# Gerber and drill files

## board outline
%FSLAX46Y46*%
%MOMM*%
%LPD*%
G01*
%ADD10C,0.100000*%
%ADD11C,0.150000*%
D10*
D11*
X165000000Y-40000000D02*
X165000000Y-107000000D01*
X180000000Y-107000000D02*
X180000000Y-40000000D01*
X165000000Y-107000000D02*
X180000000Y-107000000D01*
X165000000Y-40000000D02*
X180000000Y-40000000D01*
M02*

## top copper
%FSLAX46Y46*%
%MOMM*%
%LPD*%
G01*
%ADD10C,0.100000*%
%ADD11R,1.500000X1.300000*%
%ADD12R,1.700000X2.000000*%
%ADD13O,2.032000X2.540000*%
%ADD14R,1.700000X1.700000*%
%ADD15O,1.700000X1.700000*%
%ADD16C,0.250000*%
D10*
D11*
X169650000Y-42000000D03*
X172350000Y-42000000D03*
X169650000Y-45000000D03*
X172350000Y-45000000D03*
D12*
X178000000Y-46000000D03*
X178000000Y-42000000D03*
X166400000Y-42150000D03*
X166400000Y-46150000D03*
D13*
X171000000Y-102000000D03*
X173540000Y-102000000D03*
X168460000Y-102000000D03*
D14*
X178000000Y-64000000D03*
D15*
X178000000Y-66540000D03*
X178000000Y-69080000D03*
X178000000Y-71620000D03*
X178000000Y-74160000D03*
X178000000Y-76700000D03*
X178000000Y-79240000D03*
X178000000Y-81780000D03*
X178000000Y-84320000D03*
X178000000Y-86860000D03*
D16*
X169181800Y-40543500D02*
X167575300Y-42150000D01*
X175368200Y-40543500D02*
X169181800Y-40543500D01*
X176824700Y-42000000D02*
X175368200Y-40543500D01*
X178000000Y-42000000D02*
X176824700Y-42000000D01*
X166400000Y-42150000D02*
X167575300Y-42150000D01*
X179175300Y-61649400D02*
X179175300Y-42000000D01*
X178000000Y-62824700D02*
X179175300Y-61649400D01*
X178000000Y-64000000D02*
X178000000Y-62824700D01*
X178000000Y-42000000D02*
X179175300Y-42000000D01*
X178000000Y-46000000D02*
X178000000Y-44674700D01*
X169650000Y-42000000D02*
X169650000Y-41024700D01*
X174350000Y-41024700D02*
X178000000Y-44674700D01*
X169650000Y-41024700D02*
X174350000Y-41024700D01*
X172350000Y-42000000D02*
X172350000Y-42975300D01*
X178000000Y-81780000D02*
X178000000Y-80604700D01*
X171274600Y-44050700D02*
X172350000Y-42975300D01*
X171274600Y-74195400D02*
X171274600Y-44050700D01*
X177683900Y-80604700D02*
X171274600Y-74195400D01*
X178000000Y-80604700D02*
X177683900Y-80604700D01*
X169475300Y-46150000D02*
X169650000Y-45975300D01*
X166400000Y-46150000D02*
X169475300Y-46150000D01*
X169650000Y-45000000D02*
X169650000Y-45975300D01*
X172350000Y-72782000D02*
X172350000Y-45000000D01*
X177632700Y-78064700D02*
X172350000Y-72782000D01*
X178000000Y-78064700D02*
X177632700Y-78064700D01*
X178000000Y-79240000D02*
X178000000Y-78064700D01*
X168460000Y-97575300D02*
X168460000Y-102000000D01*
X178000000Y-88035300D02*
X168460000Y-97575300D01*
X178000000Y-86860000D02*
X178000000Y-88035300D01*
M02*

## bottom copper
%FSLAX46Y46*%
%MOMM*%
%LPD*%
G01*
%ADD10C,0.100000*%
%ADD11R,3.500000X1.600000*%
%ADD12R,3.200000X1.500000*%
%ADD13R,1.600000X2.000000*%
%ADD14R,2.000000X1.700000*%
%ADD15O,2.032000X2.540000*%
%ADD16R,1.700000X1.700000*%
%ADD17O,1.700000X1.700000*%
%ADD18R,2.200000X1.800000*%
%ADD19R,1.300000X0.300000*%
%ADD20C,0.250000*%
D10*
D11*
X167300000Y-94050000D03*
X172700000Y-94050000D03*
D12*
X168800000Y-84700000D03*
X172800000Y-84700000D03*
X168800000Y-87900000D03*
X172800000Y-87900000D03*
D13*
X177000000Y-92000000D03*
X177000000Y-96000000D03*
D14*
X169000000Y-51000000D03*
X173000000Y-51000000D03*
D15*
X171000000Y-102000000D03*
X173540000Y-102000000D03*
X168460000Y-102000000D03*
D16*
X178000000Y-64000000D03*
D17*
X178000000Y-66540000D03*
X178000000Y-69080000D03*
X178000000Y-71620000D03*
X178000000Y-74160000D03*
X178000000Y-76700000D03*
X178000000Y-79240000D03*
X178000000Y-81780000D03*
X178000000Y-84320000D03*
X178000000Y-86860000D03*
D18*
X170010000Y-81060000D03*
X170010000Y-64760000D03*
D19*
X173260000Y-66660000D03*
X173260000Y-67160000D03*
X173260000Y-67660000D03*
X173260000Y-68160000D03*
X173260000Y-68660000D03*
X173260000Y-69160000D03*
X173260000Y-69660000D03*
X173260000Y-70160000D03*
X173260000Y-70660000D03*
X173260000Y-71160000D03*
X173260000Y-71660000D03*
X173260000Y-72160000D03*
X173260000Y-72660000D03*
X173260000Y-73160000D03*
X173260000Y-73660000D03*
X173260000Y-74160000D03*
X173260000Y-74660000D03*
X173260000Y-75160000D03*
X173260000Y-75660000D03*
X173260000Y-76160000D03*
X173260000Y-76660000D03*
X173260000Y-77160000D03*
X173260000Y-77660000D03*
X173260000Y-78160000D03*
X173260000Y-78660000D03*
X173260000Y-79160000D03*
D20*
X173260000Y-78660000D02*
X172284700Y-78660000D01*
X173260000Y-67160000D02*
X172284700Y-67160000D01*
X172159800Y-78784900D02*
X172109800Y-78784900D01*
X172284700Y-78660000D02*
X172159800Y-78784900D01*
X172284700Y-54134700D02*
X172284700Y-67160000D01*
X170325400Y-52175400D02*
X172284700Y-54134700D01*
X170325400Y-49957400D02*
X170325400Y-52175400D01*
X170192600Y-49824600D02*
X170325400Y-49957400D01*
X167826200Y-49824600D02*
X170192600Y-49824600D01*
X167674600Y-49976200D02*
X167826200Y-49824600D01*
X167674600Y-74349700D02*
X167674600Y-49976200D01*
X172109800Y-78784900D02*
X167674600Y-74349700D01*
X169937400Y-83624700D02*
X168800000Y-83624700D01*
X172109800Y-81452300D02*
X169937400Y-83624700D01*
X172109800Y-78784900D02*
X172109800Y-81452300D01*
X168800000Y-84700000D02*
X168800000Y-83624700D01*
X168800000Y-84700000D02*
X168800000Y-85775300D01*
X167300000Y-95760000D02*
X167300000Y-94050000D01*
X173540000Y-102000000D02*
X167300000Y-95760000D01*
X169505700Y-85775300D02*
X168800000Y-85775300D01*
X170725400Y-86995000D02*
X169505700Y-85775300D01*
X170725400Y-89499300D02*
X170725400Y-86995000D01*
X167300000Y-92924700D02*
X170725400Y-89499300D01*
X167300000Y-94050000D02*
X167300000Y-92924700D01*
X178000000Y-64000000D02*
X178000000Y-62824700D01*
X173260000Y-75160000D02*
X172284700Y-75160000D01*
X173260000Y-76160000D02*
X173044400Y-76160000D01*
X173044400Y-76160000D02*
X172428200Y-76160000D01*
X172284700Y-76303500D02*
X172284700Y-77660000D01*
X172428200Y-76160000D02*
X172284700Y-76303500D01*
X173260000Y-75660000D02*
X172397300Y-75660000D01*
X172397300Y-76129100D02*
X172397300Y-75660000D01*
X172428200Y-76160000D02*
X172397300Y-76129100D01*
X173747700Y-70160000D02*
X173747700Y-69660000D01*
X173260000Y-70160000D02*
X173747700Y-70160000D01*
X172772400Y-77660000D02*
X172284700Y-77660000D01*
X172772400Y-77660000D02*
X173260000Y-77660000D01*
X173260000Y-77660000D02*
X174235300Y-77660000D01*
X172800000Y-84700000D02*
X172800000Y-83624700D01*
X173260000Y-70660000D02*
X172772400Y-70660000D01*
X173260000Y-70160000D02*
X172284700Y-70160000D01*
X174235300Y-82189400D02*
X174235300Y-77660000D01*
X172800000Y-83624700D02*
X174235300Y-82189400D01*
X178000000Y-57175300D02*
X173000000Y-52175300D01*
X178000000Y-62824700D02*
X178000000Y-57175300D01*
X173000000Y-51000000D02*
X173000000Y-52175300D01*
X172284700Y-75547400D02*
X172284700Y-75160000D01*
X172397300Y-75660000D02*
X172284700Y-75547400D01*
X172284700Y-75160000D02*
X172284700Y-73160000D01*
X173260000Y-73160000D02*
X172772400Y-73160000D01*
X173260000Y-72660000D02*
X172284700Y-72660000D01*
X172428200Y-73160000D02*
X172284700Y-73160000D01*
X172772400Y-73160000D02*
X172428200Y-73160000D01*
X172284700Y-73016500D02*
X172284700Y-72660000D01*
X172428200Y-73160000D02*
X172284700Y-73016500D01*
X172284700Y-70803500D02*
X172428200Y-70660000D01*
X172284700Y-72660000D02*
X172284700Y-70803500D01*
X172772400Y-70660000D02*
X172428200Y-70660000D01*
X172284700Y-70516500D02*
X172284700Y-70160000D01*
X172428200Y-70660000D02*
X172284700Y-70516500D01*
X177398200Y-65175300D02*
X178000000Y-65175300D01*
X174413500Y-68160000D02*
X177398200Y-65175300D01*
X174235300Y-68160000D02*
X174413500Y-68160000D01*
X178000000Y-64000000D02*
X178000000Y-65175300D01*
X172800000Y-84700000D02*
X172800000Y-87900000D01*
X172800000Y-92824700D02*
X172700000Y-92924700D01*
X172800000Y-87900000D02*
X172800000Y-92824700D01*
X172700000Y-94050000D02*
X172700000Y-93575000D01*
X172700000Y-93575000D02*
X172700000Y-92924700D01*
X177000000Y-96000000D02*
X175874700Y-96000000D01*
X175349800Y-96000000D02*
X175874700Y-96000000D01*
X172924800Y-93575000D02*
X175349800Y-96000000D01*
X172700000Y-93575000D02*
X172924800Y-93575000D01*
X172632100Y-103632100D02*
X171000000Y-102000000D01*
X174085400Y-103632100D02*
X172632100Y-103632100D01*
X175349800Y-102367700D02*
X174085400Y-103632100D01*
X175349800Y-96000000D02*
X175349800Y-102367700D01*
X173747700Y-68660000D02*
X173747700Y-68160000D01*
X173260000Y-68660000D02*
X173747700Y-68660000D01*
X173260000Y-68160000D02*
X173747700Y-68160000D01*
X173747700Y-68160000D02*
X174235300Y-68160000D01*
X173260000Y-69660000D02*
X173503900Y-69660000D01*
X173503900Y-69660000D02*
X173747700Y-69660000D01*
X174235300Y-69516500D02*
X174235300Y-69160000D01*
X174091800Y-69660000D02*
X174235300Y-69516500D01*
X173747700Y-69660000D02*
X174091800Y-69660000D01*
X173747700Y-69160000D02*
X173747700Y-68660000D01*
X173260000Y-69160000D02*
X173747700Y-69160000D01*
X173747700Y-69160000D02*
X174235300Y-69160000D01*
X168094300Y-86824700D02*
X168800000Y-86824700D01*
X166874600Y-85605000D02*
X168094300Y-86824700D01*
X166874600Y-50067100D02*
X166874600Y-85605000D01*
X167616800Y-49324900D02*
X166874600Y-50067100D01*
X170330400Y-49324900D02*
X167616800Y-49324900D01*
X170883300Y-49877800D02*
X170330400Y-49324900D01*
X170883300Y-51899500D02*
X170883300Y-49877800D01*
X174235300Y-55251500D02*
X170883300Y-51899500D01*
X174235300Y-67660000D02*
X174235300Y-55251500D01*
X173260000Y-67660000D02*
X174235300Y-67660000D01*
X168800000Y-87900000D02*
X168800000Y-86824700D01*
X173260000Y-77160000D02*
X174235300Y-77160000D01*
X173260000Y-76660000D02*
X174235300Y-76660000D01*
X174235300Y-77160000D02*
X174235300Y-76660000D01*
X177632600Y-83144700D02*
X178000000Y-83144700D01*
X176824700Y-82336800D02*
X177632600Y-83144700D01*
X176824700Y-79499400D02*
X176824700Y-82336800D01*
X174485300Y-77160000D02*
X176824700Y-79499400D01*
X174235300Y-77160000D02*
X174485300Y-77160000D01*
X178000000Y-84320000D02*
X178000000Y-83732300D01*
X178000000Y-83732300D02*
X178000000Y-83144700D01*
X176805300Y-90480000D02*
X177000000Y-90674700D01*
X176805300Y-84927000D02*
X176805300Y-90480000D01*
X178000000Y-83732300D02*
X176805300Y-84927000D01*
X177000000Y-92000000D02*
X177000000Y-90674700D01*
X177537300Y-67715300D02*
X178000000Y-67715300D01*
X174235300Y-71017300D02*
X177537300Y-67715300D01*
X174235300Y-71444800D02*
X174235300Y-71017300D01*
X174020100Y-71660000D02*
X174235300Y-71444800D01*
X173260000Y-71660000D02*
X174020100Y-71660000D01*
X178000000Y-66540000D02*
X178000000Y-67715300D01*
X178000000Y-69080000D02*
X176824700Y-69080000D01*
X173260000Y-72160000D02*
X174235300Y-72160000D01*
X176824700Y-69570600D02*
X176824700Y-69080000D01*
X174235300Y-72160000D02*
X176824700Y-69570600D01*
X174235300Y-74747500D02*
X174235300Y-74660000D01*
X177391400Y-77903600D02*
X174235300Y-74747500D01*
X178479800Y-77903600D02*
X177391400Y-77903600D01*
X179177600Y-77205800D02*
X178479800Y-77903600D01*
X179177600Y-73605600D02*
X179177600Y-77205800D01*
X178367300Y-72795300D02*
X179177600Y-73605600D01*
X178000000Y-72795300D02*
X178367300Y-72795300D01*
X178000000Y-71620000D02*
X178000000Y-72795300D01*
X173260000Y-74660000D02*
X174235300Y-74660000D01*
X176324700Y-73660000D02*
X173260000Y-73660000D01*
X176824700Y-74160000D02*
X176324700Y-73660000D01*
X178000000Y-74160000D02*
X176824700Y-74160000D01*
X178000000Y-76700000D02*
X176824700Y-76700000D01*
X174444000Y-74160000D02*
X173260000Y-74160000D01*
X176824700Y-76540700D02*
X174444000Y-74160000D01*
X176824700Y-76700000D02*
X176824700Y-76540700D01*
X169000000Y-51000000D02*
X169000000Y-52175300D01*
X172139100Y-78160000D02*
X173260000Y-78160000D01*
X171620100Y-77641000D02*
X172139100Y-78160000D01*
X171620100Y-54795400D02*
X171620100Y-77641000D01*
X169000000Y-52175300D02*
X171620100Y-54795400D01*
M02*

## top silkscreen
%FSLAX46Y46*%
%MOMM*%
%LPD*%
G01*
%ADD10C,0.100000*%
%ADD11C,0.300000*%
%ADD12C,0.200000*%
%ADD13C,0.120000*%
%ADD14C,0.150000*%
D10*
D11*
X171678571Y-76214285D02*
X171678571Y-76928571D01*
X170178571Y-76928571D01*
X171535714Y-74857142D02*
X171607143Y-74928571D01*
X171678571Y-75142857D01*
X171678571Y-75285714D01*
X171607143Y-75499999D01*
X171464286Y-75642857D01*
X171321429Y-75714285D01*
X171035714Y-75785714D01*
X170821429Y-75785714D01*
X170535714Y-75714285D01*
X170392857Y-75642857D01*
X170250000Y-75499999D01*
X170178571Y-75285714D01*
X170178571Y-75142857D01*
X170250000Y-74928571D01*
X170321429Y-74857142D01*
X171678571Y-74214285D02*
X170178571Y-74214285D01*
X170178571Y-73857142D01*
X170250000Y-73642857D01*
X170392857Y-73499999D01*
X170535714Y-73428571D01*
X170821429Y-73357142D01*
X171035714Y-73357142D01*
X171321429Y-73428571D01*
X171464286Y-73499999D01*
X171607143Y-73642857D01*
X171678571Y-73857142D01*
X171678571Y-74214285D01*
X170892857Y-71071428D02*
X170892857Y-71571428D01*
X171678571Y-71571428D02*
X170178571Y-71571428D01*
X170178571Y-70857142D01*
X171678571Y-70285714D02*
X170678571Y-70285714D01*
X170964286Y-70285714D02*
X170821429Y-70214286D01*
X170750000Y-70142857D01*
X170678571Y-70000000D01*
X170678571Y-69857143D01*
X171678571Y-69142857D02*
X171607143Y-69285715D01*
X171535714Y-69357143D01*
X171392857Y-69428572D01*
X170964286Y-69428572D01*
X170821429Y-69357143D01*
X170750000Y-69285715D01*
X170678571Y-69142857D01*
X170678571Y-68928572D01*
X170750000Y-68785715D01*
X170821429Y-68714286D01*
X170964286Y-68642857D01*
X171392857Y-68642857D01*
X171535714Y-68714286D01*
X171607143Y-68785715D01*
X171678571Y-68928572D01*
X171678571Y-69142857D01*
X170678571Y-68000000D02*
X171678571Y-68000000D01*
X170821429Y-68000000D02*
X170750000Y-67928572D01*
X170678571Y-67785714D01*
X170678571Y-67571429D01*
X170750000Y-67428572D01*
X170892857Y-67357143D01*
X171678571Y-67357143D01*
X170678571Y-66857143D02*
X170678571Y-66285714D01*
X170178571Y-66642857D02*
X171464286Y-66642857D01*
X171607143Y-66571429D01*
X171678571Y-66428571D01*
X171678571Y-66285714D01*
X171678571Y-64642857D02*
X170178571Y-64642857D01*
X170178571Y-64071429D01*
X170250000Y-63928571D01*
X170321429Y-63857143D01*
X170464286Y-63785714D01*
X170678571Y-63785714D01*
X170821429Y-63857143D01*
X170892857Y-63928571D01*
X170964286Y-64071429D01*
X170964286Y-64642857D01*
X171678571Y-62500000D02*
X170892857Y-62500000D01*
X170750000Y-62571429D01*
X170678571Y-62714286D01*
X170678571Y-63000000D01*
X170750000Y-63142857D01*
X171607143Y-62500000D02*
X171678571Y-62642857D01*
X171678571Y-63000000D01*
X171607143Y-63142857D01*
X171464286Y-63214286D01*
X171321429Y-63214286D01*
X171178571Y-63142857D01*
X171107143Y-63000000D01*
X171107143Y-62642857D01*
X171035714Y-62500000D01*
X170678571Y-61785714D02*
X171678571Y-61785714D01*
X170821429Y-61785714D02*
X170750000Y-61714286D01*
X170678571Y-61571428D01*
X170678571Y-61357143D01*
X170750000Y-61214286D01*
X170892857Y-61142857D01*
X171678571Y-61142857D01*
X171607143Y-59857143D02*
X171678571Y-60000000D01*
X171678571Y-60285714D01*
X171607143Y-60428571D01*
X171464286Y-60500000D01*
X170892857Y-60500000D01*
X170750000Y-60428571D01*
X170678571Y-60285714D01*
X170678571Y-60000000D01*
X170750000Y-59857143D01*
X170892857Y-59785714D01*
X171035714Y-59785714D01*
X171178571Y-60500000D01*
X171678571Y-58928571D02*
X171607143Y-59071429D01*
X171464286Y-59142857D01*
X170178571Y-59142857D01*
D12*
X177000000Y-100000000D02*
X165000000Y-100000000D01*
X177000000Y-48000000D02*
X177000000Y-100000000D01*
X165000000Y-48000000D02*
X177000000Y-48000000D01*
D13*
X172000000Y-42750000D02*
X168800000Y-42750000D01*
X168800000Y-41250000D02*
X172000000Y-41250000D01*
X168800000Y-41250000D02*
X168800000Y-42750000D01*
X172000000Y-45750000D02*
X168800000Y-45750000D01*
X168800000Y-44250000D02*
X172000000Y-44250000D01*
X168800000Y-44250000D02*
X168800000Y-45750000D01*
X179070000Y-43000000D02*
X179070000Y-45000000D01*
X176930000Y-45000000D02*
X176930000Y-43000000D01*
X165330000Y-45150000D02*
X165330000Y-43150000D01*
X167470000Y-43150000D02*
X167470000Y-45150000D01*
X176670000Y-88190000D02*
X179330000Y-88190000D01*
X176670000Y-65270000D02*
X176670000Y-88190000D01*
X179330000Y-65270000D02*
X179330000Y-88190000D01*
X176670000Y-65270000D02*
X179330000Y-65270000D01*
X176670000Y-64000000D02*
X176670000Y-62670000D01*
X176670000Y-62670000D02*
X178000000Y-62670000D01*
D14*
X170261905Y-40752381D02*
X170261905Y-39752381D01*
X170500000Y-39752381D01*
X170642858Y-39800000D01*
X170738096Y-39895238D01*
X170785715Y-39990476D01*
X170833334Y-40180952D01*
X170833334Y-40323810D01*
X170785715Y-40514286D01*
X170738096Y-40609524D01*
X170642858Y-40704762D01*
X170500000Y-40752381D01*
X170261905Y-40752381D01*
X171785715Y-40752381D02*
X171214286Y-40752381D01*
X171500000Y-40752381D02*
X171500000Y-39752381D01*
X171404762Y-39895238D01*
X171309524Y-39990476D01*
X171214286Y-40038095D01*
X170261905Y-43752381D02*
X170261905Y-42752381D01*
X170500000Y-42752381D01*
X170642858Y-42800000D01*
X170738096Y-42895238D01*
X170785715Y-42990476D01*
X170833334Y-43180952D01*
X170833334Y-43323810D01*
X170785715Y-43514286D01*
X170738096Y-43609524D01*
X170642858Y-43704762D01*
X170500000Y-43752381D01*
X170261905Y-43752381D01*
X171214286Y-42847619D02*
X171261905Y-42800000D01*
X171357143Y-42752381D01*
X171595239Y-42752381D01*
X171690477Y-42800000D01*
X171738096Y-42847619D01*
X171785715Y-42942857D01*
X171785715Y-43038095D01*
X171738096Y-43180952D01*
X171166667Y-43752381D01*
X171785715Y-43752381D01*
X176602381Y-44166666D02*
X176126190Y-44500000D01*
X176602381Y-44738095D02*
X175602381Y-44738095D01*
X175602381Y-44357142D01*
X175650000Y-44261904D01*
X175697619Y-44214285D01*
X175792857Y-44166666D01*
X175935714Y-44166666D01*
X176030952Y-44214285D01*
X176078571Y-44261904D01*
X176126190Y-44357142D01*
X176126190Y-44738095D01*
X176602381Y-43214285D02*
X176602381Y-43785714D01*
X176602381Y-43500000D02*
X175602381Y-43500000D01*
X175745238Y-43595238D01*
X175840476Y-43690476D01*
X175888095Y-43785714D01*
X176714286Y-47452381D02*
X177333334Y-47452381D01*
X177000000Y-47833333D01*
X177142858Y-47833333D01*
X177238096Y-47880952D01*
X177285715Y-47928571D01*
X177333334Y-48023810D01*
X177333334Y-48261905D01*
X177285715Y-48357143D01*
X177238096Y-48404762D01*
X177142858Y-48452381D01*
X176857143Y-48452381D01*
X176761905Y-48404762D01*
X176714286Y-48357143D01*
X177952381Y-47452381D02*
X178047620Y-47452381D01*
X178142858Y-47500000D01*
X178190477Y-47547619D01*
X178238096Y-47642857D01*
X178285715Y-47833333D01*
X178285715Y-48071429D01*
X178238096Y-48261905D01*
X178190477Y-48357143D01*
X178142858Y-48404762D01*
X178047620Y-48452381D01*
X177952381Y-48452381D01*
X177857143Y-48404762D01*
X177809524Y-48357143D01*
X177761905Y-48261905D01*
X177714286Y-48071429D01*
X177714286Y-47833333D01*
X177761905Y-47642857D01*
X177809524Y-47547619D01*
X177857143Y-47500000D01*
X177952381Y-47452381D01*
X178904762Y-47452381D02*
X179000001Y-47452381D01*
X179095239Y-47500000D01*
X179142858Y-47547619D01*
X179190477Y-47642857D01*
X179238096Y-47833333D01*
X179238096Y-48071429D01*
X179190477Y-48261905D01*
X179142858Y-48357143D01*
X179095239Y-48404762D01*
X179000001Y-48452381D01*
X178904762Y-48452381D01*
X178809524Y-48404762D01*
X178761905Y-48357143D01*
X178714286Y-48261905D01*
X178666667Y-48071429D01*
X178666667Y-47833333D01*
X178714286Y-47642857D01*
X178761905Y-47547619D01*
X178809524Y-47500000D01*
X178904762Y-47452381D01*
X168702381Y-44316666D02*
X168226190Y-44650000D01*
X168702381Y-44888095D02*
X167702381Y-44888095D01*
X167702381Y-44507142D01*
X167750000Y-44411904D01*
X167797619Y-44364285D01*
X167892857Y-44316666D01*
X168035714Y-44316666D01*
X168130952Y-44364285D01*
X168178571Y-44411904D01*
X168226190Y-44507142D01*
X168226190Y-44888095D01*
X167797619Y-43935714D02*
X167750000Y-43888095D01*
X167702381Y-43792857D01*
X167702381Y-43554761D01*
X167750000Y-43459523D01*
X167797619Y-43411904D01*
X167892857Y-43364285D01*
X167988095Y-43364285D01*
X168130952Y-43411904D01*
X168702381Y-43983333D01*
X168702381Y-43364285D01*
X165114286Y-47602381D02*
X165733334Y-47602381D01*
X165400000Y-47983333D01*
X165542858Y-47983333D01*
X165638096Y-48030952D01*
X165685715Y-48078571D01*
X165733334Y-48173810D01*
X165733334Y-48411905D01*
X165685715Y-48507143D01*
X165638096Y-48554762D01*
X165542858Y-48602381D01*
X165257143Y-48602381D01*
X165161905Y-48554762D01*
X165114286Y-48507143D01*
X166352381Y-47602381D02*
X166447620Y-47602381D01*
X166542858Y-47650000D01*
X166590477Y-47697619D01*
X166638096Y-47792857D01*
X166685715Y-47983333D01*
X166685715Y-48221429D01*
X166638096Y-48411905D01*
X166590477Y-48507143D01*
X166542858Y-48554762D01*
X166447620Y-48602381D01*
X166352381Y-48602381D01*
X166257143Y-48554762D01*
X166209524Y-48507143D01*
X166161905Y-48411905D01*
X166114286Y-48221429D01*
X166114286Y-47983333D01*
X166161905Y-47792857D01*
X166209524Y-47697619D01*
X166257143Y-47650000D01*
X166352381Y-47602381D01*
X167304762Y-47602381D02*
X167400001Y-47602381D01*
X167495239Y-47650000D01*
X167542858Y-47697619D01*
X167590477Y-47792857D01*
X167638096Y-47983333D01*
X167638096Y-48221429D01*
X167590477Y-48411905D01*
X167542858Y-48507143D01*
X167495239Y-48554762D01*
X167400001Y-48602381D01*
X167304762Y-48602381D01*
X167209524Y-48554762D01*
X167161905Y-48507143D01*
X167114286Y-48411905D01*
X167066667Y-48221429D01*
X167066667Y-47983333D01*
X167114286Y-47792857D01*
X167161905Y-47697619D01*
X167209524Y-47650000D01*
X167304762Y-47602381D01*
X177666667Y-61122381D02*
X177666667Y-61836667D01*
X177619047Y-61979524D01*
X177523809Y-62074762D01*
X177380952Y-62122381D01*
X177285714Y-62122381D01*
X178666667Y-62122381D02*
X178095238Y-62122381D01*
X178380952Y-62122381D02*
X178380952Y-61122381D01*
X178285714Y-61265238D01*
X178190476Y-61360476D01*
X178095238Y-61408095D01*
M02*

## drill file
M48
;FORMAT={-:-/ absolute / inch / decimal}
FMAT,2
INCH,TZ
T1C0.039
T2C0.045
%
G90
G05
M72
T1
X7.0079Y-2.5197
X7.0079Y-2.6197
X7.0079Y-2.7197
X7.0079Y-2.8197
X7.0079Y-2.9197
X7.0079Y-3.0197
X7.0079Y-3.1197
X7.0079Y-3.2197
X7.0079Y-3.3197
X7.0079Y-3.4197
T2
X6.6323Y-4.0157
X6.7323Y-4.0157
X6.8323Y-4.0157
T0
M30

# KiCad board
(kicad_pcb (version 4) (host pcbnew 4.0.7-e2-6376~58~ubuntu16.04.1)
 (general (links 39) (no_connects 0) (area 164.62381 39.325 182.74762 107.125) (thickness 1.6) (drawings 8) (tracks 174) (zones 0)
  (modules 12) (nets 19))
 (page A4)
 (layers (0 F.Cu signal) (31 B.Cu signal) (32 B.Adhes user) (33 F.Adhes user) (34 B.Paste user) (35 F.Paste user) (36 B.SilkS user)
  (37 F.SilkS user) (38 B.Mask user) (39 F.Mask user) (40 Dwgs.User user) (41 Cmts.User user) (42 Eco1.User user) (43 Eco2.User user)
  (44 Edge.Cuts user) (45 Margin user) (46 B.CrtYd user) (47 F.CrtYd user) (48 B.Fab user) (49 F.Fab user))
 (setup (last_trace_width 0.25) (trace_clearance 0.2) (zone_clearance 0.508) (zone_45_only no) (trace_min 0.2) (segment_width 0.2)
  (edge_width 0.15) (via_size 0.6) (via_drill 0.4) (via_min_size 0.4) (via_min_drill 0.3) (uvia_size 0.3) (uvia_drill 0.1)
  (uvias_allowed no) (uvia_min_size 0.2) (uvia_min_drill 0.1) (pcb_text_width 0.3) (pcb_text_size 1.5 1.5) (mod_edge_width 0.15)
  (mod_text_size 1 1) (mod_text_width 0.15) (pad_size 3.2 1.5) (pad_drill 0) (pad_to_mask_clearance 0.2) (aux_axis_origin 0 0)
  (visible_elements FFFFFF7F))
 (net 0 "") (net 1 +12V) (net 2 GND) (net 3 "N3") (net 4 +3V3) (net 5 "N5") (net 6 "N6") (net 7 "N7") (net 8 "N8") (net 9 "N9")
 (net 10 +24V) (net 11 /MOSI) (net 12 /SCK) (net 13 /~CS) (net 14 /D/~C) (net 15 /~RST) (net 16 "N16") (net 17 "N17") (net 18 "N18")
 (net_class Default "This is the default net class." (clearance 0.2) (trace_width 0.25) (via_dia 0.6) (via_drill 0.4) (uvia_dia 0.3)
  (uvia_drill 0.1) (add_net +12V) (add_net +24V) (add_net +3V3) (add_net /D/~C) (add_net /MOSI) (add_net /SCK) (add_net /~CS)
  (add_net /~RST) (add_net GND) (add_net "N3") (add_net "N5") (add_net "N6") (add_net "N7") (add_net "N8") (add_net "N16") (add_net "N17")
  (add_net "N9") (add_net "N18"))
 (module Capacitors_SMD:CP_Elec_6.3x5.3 (layer B.Cu) (at 170 94.05)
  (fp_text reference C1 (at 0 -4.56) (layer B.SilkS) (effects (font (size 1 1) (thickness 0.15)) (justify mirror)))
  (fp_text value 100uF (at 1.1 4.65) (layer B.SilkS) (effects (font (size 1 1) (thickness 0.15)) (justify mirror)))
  (pad 1 smd rect (at -2.7 0 180) (size 3.5 1.6) (layers B.Cu B.Paste B.Mask) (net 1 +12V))
  (pad 2 smd rect (at 2.7 0 180) (size 3.5 1.6) (layers B.Cu B.Paste B.Mask) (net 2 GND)))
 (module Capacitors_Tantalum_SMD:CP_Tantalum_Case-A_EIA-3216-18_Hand (layer B.Cu) (at 170.8 84.7)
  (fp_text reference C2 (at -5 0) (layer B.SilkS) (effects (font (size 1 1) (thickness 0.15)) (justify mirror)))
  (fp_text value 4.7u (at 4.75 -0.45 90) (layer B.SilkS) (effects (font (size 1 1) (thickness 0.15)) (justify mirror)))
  (pad 1 smd rect (at -2 0) (size 3.2 1.5) (layers B.Cu B.Paste B.Mask) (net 1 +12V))
  (pad 2 smd rect (at 2 0) (size 3.2 1.5) (layers B.Cu B.Paste B.Mask) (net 2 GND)))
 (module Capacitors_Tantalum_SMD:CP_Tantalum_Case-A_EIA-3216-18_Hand (layer B.Cu) (at 170.8 87.9)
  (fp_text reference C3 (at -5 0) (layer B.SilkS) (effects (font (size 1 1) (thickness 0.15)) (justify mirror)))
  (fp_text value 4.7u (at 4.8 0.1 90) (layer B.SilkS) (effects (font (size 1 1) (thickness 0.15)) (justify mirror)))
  (pad 1 smd rect (at -2 0) (size 3.2 1.5) (layers B.Cu B.Paste B.Mask) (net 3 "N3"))
  (pad 2 smd rect (at 2 0) (size 3.2 1.5) (layers B.Cu B.Paste B.Mask) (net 2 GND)))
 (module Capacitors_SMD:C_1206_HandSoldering (layer B.Cu) (at 177 94 270)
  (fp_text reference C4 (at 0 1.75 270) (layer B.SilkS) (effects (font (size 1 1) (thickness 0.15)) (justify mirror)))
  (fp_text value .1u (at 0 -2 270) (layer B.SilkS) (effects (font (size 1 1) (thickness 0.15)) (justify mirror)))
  (pad 1 smd rect (at -2 0 270) (size 2 1.6) (layers B.Cu B.Paste B.Mask) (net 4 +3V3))
  (pad 2 smd rect (at 2 0 270) (size 2 1.6) (layers B.Cu B.Paste B.Mask) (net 2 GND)))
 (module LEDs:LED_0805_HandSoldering (layer F.Cu) (at 171 42)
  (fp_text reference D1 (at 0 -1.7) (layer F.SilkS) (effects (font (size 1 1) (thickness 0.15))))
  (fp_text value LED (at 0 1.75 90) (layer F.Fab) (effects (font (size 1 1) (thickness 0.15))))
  (fp_line (start 1 0.75) (end -2.2 0.75) (layer F.SilkS) (width 0.12))
  (fp_line (start -2.2 -0.75) (end 1 -0.75) (layer F.SilkS) (width 0.12))
  (fp_line (start -2.2 -0.75) (end -2.2 0.75) (layer F.SilkS) (width 0.12))
  (pad 1 smd rect (at -1.35 0) (size 1.5 1.3) (layers F.Cu F.Paste F.Mask) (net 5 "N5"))
  (pad 2 smd rect (at 1.35 0) (size 1.5 1.3) (layers F.Cu F.Paste F.Mask) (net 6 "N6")))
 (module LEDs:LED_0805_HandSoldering (layer F.Cu) (at 171 45)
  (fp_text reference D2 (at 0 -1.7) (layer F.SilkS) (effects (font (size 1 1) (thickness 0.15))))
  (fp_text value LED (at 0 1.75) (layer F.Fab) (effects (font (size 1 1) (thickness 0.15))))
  (fp_line (start 1 0.75) (end -2.2 0.75) (layer F.SilkS) (width 0.12))
  (fp_line (start -2.2 -0.75) (end 1 -0.75) (layer F.SilkS) (width 0.12))
  (fp_line (start -2.2 -0.75) (end -2.2 0.75) (layer F.SilkS) (width 0.12))
  (pad 1 smd rect (at -1.35 0) (size 1.5 1.3) (layers F.Cu F.Paste F.Mask) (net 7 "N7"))
  (pad 2 smd rect (at 1.35 0) (size 1.5 1.3) (layers F.Cu F.Paste F.Mask) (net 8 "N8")))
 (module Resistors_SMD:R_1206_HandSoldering (layer F.Cu) (at 178 44 90)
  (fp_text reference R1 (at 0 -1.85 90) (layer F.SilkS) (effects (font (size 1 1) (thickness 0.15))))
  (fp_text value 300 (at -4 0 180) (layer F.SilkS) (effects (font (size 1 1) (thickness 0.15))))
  (fp_line (start 1 1.07) (end -1 1.07) (layer F.SilkS) (width 0.12))
  (fp_line (start -1 -1.07) (end 1 -1.07) (layer F.SilkS) (width 0.12))
  (pad 1 smd rect (at -2 0 90) (size 2 1.7) (layers F.Cu F.Paste F.Mask) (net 5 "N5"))
  (pad 2 smd rect (at 2 0 90) (size 2 1.7) (layers F.Cu F.Paste F.Mask) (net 2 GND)))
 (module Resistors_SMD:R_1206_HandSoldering (layer F.Cu) (at 166.4 44.15 270)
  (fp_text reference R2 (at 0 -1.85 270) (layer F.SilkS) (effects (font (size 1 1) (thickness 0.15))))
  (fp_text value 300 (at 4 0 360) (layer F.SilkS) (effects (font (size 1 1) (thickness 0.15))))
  (fp_line (start 1 1.07) (end -1 1.07) (layer F.SilkS) (width 0.12))
  (fp_line (start -1 -1.07) (end 1 -1.07) (layer F.SilkS) (width 0.12))
  (pad 1 smd rect (at -2 0 270) (size 2 1.7) (layers F.Cu F.Paste F.Mask) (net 2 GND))
  (pad 2 smd rect (at 2 0 270) (size 2 1.7) (layers F.Cu F.Paste F.Mask) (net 7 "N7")))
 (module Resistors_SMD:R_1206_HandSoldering (layer B.Cu) (at 171 51)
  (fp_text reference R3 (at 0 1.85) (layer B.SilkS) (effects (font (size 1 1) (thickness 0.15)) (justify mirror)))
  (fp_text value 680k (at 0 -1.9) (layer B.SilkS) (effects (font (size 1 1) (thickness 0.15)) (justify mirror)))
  (pad 1 smd rect (at -2 0) (size 2 1.7) (layers B.Cu B.Paste B.Mask) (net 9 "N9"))
  (pad 2 smd rect (at 2 0) (size 2 1.7) (layers B.Cu B.Paste B.Mask) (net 2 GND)))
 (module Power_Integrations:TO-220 (layer B.Cu) (at 171 102)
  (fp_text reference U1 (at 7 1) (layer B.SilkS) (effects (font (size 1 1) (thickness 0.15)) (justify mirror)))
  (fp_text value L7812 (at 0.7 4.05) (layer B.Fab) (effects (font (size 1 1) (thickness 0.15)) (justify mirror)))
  (pad 2 thru_hole oval (at 0 0) (size 2.032 2.54) (drill 1.143) (layers *.Cu *.Mask) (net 2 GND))
  (pad 3 thru_hole oval (at 2.54 0) (size 2.032 2.54) (drill 1.143) (layers *.Cu *.Mask) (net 1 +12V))
  (pad 1 thru_hole oval (at -2.54 0) (size 2.032 2.54) (drill 1.143) (layers *.Cu *.Mask) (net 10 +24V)))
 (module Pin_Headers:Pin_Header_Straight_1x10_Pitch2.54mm (layer F.Cu) (at 178 64)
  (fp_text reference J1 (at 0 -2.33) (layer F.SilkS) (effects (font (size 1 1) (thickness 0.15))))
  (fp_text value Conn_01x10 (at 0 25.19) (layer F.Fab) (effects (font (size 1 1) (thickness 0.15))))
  (fp_line (start -1.33 24.19) (end 1.33 24.19) (layer F.SilkS) (width 0.12))
  (fp_line (start -1.33 1.27) (end -1.33 24.19) (layer F.SilkS) (width 0.12))
  (fp_line (start 1.33 1.27) (end 1.33 24.19) (layer F.SilkS) (width 0.12))
  (fp_line (start -1.33 1.27) (end 1.33 1.27) (layer F.SilkS) (width 0.12))
  (fp_line (start -1.33 0) (end -1.33 -1.33) (layer F.SilkS) (width 0.12))
  (fp_line (start -1.33 -1.33) (end 0 -1.33) (layer F.SilkS) (width 0.12))
  (pad 1 thru_hole rect (at 0 0) (size 1.7 1.7) (drill 1) (layers *.Cu *.Mask) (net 2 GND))
  (pad 2 thru_hole oval (at 0 2.54) (size 1.7 1.7) (drill 1) (layers *.Cu *.Mask) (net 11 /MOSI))
  (pad 3 thru_hole oval (at 0 5.08) (size 1.7 1.7) (drill 1) (layers *.Cu *.Mask) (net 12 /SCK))
  (pad 4 thru_hole oval (at 0 7.62) (size 1.7 1.7) (drill 1) (layers *.Cu *.Mask) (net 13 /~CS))
  (pad 5 thru_hole oval (at 0 10.16) (size 1.7 1.7) (drill 1) (layers *.Cu *.Mask) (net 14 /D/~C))
  (pad 6 thru_hole oval (at 0 12.7) (size 1.7 1.7) (drill 1) (layers *.Cu *.Mask) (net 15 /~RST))
  (pad 7 thru_hole oval (at 0 15.24) (size 1.7 1.7) (drill 1) (layers *.Cu *.Mask) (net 8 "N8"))
  (pad 8 thru_hole oval (at 0 17.78) (size 1.7 1.7) (drill 1) (layers *.Cu *.Mask) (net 6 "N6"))
  (pad 9 thru_hole oval (at 0 20.32) (size 1.7 1.7) (drill 1) (layers *.Cu *.Mask) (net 4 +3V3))
  (pad 10 thru_hole oval (at 0 22.86) (size 1.7 1.7) (drill 1) (layers *.Cu *.Mask) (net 10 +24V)))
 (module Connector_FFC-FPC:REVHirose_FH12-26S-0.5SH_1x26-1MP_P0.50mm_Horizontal (layer B.Cu) (at 171.41 74.18 90)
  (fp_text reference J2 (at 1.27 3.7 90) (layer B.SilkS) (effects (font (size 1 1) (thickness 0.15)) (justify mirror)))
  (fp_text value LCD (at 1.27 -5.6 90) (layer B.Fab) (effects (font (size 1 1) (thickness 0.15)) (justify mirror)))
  (pad MP smd rect (at -6.88 -1.4 90) (size 1.8 2.2) (layers B.Cu B.Paste B.Mask))
  (pad MP smd rect (at 9.42 -1.4 90) (size 1.8 2.2) (layers B.Cu B.Paste B.Mask))
  (pad 1 smd rect (at 7.52 1.85 90) (size 0.3 1.3) (layers B.Cu B.Paste B.Mask) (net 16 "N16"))
  (pad 2 smd rect (at 7.02 1.85 90) (size 0.3 1.3) (layers B.Cu B.Paste B.Mask) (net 1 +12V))
  (pad 3 smd rect (at 6.52 1.85 90) (size 0.3 1.3) (layers B.Cu B.Paste B.Mask) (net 3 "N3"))
  (pad 4 smd rect (at 6.02 1.85 90) (size 0.3 1.3) (layers B.Cu B.Paste B.Mask) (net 2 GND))
  (pad 5 smd rect (at 5.52 1.85 90) (size 0.3 1.3) (layers B.Cu B.Paste B.Mask) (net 2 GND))
  (pad 6 smd rect (at 5.02 1.85 90) (size 0.3 1.3) (layers B.Cu B.Paste B.Mask) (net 2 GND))
  (pad 7 smd rect (at 4.52 1.85 90) (size 0.3 1.3) (layers B.Cu B.Paste B.Mask) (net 2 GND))
  (pad 8 smd rect (at 4.02 1.85 90) (size 0.3 1.3) (layers B.Cu B.Paste B.Mask) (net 2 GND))
  (pad 9 smd rect (at 3.52 1.85 90) (size 0.3 1.3) (layers B.Cu B.Paste B.Mask) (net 2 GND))
  (pad 10 smd rect (at 3.02 1.85 90) (size 0.3 1.3) (layers B.Cu B.Paste B.Mask) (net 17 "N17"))
  (pad 11 smd rect (at 2.52 1.85 90) (size 0.3 1.3) (layers B.Cu B.Paste B.Mask) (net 11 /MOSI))
  (pad 12 smd rect (at 2.02 1.85 90) (size 0.3 1.3) (layers B.Cu B.Paste B.Mask) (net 12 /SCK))
  (pad 13 smd rect (at 1.52 1.85 90) (size 0.3 1.3) (layers B.Cu B.Paste B.Mask) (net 2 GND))
  (pad 14 smd rect (at 1.02 1.85 90) (size 0.3 1.3) (layers B.Cu B.Paste B.Mask) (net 2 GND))
  (pad 15 smd rect (at 0.52 1.85 90) (size 0.3 1.3) (layers B.Cu B.Paste B.Mask) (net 14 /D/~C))
  (pad 16 smd rect (at 0.02 1.85 90) (size 0.3 1.3) (layers B.Cu B.Paste B.Mask) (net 15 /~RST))
  (pad 17 smd rect (at -0.48 1.85 90) (size 0.3 1.3) (layers B.Cu B.Paste B.Mask) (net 13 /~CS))
  (pad 18 smd rect (at -0.98 1.85 90) (size 0.3 1.3) (layers B.Cu B.Paste B.Mask) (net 2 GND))
  (pad 19 smd rect (at -1.48 1.85 90) (size 0.3 1.3) (layers B.Cu B.Paste B.Mask) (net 2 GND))
  (pad 20 smd rect (at -1.98 1.85 90) (size 0.3 1.3) (layers B.Cu B.Paste B.Mask) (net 2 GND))
  (pad 21 smd rect (at -2.48 1.85 90) (size 0.3 1.3) (layers B.Cu B.Paste B.Mask) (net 4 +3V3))
  (pad 22 smd rect (at -2.98 1.85 90) (size 0.3 1.3) (layers B.Cu B.Paste B.Mask) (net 4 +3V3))
  (pad 23 smd rect (at -3.48 1.85 90) (size 0.3 1.3) (layers B.Cu B.Paste B.Mask) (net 2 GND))
  (pad 24 smd rect (at -3.98 1.85 90) (size 0.3 1.3) (layers B.Cu B.Paste B.Mask) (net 9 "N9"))
  (pad 25 smd rect (at -4.48 1.85 90) (size 0.3 1.3) (layers B.Cu B.Paste B.Mask) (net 1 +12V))
  (pad 26 smd rect (at -4.98 1.85 90) (size 0.3 1.3) (layers B.Cu B.Paste B.Mask) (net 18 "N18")))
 (gr_line (start 165 40) (end 165 107) (angle 90) (layer Edge.Cuts) (width 0.15))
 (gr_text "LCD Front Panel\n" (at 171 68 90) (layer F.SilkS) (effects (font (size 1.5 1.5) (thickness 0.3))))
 (gr_line (start 180 107) (end 180 40) (angle 90) (layer Edge.Cuts) (width 0.15))
 (gr_line (start 165 107) (end 180 107) (angle 90) (layer Edge.Cuts) (width 0.15))
 (gr_line (start 177 100) (end 165 100) (angle 90) (layer F.SilkS) (width 0.2))
 (gr_line (start 177 48) (end 177 100) (angle 90) (layer F.SilkS) (width 0.2))
 (gr_line (start 165 48) (end 177 48) (angle 90) (layer F.SilkS) (width 0.2))
 (gr_line (start 165 40) (end 180 40) (angle 90) (layer Edge.Cuts) (width 0.15))
 (segment (start 173.26 78.66) (end 172.2847 78.66) (width 0.25) (layer B.Cu) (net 1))
 (segment (start 173.26 67.16) (end 172.2847 67.16) (width 0.25) (layer B.Cu) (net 1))
 (segment (start 172.1598 78.7849) (end 172.1098 78.7849) (width 0.25) (layer B.Cu) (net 1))
 (segment (start 172.2847 78.66) (end 172.1598 78.7849) (width 0.25) (layer B.Cu) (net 1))
 (segment (start 172.2847 54.1347) (end 172.2847 67.16) (width 0.25) (layer B.Cu) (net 1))
 (segment (start 170.3254 52.1754) (end 172.2847 54.1347) (width 0.25) (layer B.Cu) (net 1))
 (segment (start 170.3254 49.9574) (end 170.3254 52.1754) (width 0.25) (layer B.Cu) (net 1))
 (segment (start 170.1926 49.8246) (end 170.3254 49.9574) (width 0.25) (layer B.Cu) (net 1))
 (segment (start 167.8262 49.8246) (end 170.1926 49.8246) (width 0.25) (layer B.Cu) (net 1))
 (segment (start 167.6746 49.9762) (end 167.8262 49.8246) (width 0.25) (layer B.Cu) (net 1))
 (segment (start 167.6746 74.3497) (end 167.6746 49.9762) (width 0.25) (layer B.Cu) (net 1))
 (segment (start 172.1098 78.7849) (end 167.6746 74.3497) (width 0.25) (layer B.Cu) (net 1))
 (segment (start 169.9374 83.6247) (end 168.8 83.6247) (width 0.25) (layer B.Cu) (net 1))
 (segment (start 172.1098 81.4523) (end 169.9374 83.6247) (width 0.25) (layer B.Cu) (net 1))
 (segment (start 172.1098 78.7849) (end 172.1098 81.4523) (width 0.25) (layer B.Cu) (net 1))
 (segment (start 168.8 84.7) (end 168.8 83.6247) (width 0.25) (layer B.Cu) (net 1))
 (segment (start 168.8 84.7) (end 168.8 85.7753) (width 0.25) (layer B.Cu) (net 1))
 (segment (start 167.3 95.76) (end 167.3 94.05) (width 0.25) (layer B.Cu) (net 1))
 (segment (start 173.54 102) (end 167.3 95.76) (width 0.25) (layer B.Cu) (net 1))
 (segment (start 169.5057 85.7753) (end 168.8 85.7753) (width 0.25) (layer B.Cu) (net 1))
 (segment (start 170.7254 86.995) (end 169.5057 85.7753) (width 0.25) (layer B.Cu) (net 1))
 (segment (start 170.7254 89.4993) (end 170.7254 86.995) (width 0.25) (layer B.Cu) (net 1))
 (segment (start 167.3 92.9247) (end 170.7254 89.4993) (width 0.25) (layer B.Cu) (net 1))
 (segment (start 167.3 94.05) (end 167.3 92.9247) (width 0.25) (layer B.Cu) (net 1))
 (segment (start 178 64) (end 178 62.8247) (width 0.25) (layer B.Cu) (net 2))
 (segment (start 173.26 75.16) (end 172.2847 75.16) (width 0.25) (layer B.Cu) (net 2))
 (segment (start 169.1818 40.5435) (end 167.5753 42.15) (width 0.25) (layer F.Cu) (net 2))
 (segment (start 175.3682 40.5435) (end 169.1818 40.5435) (width 0.25) (layer F.Cu) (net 2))
 (segment (start 176.8247 42) (end 175.3682 40.5435) (width 0.25) (layer F.Cu) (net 2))
 (segment (start 178 42) (end 176.8247 42) (width 0.25) (layer F.Cu) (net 2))
 (segment (start 166.4 42.15) (end 167.5753 42.15) (width 0.25) (layer F.Cu) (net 2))
 (segment (start 173.26 76.16) (end 173.0444 76.16) (width 0.25) (layer B.Cu) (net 2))
 (segment (start 173.0444 76.16) (end 172.4282 76.16) (width 0.25) (layer B.Cu) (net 2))
 (segment (start 172.2847 76.3035) (end 172.2847 77.66) (width 0.25) (layer B.Cu) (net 2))
 (segment (start 172.4282 76.16) (end 172.2847 76.3035) (width 0.25) (layer B.Cu) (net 2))
 (segment (start 173.26 75.66) (end 172.3973 75.66) (width 0.25) (layer B.Cu) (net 2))
 (segment (start 172.3973 76.1291) (end 172.3973 75.66) (width 0.25) (layer B.Cu) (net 2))
 (segment (start 172.4282 76.16) (end 172.3973 76.1291) (width 0.25) (layer B.Cu) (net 2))
 (segment (start 173.7477 70.16) (end 173.7477 69.66) (width 0.25) (layer B.Cu) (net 2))
 (segment (start 173.26 70.16) (end 173.7477 70.16) (width 0.25) (layer B.Cu) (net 2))
 (segment (start 172.7724 77.66) (end 172.2847 77.66) (width 0.25) (layer B.Cu) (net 2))
 (segment (start 172.7724 77.66) (end 173.26 77.66) (width 0.25) (layer B.Cu) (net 2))
 (segment (start 173.26 77.66) (end 174.2353 77.66) (width 0.25) (layer B.Cu) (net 2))
 (segment (start 172.8 84.7) (end 172.8 83.6247) (width 0.25) (layer B.Cu) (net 2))
 (segment (start 173.26 70.66) (end 172.7724 70.66) (width 0.25) (layer B.Cu) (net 2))
 (segment (start 173.26 70.16) (end 172.2847 70.16) (width 0.25) (layer B.Cu) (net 2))
 (segment (start 174.2353 82.1894) (end 174.2353 77.66) (width 0.25) (layer B.Cu) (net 2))
 (segment (start 172.8 83.6247) (end 174.2353 82.1894) (width 0.25) (layer B.Cu) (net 2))
 (segment (start 178 57.1753) (end 173 52.1753) (width 0.25) (layer B.Cu) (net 2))
 (segment (start 178 62.8247) (end 178 57.1753) (width 0.25) (layer B.Cu) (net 2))
 (segment (start 173 51) (end 173 52.1753) (width 0.25) (layer B.Cu) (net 2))
 (segment (start 172.2847 75.5474) (end 172.2847 75.16) (width 0.25) (layer B.Cu) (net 2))
 (segment (start 172.3973 75.66) (end 172.2847 75.5474) (width 0.25) (layer B.Cu) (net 2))
 (segment (start 172.2847 75.16) (end 172.2847 73.16) (width 0.25) (layer B.Cu) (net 2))
 (segment (start 173.26 73.16) (end 172.7724 73.16) (width 0.25) (layer B.Cu) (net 2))
 (segment (start 173.26 72.66) (end 172.2847 72.66) (width 0.25) (layer B.Cu) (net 2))
 (segment (start 172.4282 73.16) (end 172.2847 73.16) (width 0.25) (layer B.Cu) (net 2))
 (segment (start 172.7724 73.16) (end 172.4282 73.16) (width 0.25) (layer B.Cu) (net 2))
 (segment (start 172.2847 73.0165) (end 172.2847 72.66) (width 0.25) (layer B.Cu) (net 2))
 (segment (start 172.4282 73.16) (end 172.2847 73.0165) (width 0.25) (layer B.Cu) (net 2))
 (segment (start 172.2847 70.8035) (end 172.4282 70.66) (width 0.25) (layer B.Cu) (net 2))
 (segment (start 172.2847 72.66) (end 172.2847 70.8035) (width 0.25) (layer B.Cu) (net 2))
 (segment (start 172.7724 70.66) (end 172.4282 70.66) (width 0.25) (layer B.Cu) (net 2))
 (segment (start 172.2847 70.5165) (end 172.2847 70.16) (width 0.25) (layer B.Cu) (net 2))
 (segment (start 172.4282 70.66) (end 172.2847 70.5165) (width 0.25) (layer B.Cu) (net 2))
 (segment (start 177.3982 65.1753) (end 178 65.1753) (width 0.25) (layer B.Cu) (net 2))
 (segment (start 174.4135 68.16) (end 177.3982 65.1753) (width 0.25) (layer B.Cu) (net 2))
 (segment (start 174.2353 68.16) (end 174.4135 68.16) (width 0.25) (layer B.Cu) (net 2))
 (segment (start 178 64) (end 178 65.1753) (width 0.25) (layer B.Cu) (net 2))
 (segment (start 172.8 84.7) (end 172.8 87.9) (width 0.25) (layer B.Cu) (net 2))
 (segment (start 172.8 92.8247) (end 172.7 92.9247) (width 0.25) (layer B.Cu) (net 2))
 (segment (start 172.8 87.9) (end 172.8 92.8247) (width 0.25) (layer B.Cu) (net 2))
 (segment (start 172.7 94.05) (end 172.7 93.575) (width 0.25) (layer B.Cu) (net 2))
 (segment (start 172.7 93.575) (end 172.7 92.9247) (width 0.25) (layer B.Cu) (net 2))
 (segment (start 177 96) (end 175.8747 96) (width 0.25) (layer B.Cu) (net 2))
 (segment (start 179.1753 61.6494) (end 179.1753 42) (width 0.25) (layer F.Cu) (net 2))
 (segment (start 178 62.8247) (end 179.1753 61.6494) (width 0.25) (layer F.Cu) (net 2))
 (segment (start 178 64) (end 178 62.8247) (width 0.25) (layer F.Cu) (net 2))
 (segment (start 178 42) (end 179.1753 42) (width 0.25) (layer F.Cu) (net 2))
 (segment (start 175.3498 96) (end 175.8747 96) (width 0.25) (layer B.Cu) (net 2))
 (segment (start 172.9248 93.575) (end 175.3498 96) (width 0.25) (layer B.Cu) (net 2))
 (segment (start 172.7 93.575) (end 172.9248 93.575) (width 0.25) (layer B.Cu) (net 2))
 (segment (start 172.6321 103.6321) (end 171 102) (width 0.25) (layer B.Cu) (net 2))
 (segment (start 174.0854 103.6321) (end 172.6321 103.6321) (width 0.25) (layer B.Cu) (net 2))
 (segment (start 175.3498 102.3677) (end 174.0854 103.6321) (width 0.25) (layer B.Cu) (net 2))
 (segment (start 175.3498 96) (end 175.3498 102.3677) (width 0.25) (layer B.Cu) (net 2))
 (segment (start 173.7477 68.66) (end 173.7477 68.16) (width 0.25) (layer B.Cu) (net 2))
 (segment (start 173.26 68.66) (end 173.7477 68.66) (width 0.25) (layer B.Cu) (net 2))
 (segment (start 173.26 68.16) (end 173.7477 68.16) (width 0.25) (layer B.Cu) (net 2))
 (segment (start 173.7477 68.16) (end 174.2353 68.16) (width 0.25) (layer B.Cu) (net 2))
 (segment (start 173.26 69.66) (end 173.5039 69.66) (width 0.25) (layer B.Cu) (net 2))
 (segment (start 173.5039 69.66) (end 173.7477 69.66) (width 0.25) (layer B.Cu) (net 2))
 (segment (start 174.2353 69.5165) (end 174.2353 69.16) (width 0.25) (layer B.Cu) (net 2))
 (segment (start 174.0918 69.66) (end 174.2353 69.5165) (width 0.25) (layer B.Cu) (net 2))
 (segment (start 173.7477 69.66) (end 174.0918 69.66) (width 0.25) (layer B.Cu) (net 2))
 (segment (start 173.7477 69.16) (end 173.7477 68.66) (width 0.25) (layer B.Cu) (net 2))
 (segment (start 173.26 69.16) (end 173.7477 69.16) (width 0.25) (layer B.Cu) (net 2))
 (segment (start 173.7477 69.16) (end 174.2353 69.16) (width 0.25) (layer B.Cu) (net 2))
 (segment (start 168.0943 86.8247) (end 168.8 86.8247) (width 0.25) (layer B.Cu) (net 3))
 (segment (start 166.8746 85.605) (end 168.0943 86.8247) (width 0.25) (layer B.Cu) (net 3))
 (segment (start 166.8746 50.0671) (end 166.8746 85.605) (width 0.25) (layer B.Cu) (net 3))
 (segment (start 167.6168 49.3249) (end 166.8746 50.0671) (width 0.25) (layer B.Cu) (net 3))
 (segment (start 170.3304 49.3249) (end 167.6168 49.3249) (width 0.25) (layer B.Cu) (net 3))
 (segment (start 170.8833 49.8778) (end 170.3304 49.3249) (width 0.25) (layer B.Cu) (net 3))
 (segment (start 170.8833 51.8995) (end 170.8833 49.8778) (width 0.25) (layer B.Cu) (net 3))
 (segment (start 174.2353 55.2515) (end 170.8833 51.8995) (width 0.25) (layer B.Cu) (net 3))
 (segment (start 174.2353 67.66) (end 174.2353 55.2515) (width 0.25) (layer B.Cu) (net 3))
 (segment (start 173.26 67.66) (end 174.2353 67.66) (width 0.25) (layer B.Cu) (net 3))
 (segment (start 168.8 87.9) (end 168.8 86.8247) (width 0.25) (layer B.Cu) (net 3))
 (segment (start 173.26 77.16) (end 174.2353 77.16) (width 0.25) (layer B.Cu) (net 4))
 (segment (start 173.26 76.66) (end 174.2353 76.66) (width 0.25) (layer B.Cu) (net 4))
 (segment (start 174.2353 77.16) (end 174.2353 76.66) (width 0.25) (layer B.Cu) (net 4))
 (segment (start 177.6326 83.1447) (end 178 83.1447) (width 0.25) (layer B.Cu) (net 4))
 (segment (start 176.8247 82.3368) (end 177.6326 83.1447) (width 0.25) (layer B.Cu) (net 4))
 (segment (start 176.8247 79.4994) (end 176.8247 82.3368) (width 0.25) (layer B.Cu) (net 4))
 (segment (start 174.4853 77.16) (end 176.8247 79.4994) (width 0.25) (layer B.Cu) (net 4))
 (segment (start 174.2353 77.16) (end 174.4853 77.16) (width 0.25) (layer B.Cu) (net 4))
 (segment (start 178 84.32) (end 178 83.7323) (width 0.25) (layer B.Cu) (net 4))
 (segment (start 178 83.7323) (end 178 83.1447) (width 0.25) (layer B.Cu) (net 4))
 (segment (start 176.8053 90.48) (end 177 90.6747) (width 0.25) (layer B.Cu) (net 4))
 (segment (start 176.8053 84.927) (end 176.8053 90.48) (width 0.25) (layer B.Cu) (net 4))
 (segment (start 178 83.7323) (end 176.8053 84.927) (width 0.25) (layer B.Cu) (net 4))
 (segment (start 177 92) (end 177 90.6747) (width 0.25) (layer B.Cu) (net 4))
 (segment (start 178 46) (end 178 44.6747) (width 0.25) (layer F.Cu) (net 5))
 (segment (start 169.65 42) (end 169.65 41.0247) (width 0.25) (layer F.Cu) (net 5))
 (segment (start 174.35 41.0247) (end 178 44.6747) (width 0.25) (layer F.Cu) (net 5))
 (segment (start 169.65 41.0247) (end 174.35 41.0247) (width 0.25) (layer F.Cu) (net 5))
 (segment (start 172.35 42) (end 172.35 42.9753) (width 0.25) (layer F.Cu) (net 6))
 (segment (start 178 81.78) (end 178 80.6047) (width 0.25) (layer F.Cu) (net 6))
 (segment (start 171.2746 44.0507) (end 172.35 42.9753) (width 0.25) (layer F.Cu) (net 6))
 (segment (start 171.2746 74.1954) (end 171.2746 44.0507) (width 0.25) (layer F.Cu) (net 6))
 (segment (start 177.6839 80.6047) (end 171.2746 74.1954) (width 0.25) (layer F.Cu) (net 6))
 (segment (start 178 80.6047) (end 177.6839 80.6047) (width 0.25) (layer F.Cu) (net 6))
 (segment (start 169.4753 46.15) (end 169.65 45.9753) (width 0.25) (layer F.Cu) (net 7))
 (segment (start 166.4 46.15) (end 169.4753 46.15) (width 0.25) (layer F.Cu) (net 7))
 (segment (start 169.65 45) (end 169.65 45.9753) (width 0.25) (layer F.Cu) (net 7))
 (segment (start 172.35 72.782) (end 172.35 45) (width 0.25) (layer F.Cu) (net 8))
 (segment (start 177.6327 78.0647) (end 172.35 72.782) (width 0.25) (layer F.Cu) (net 8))
 (segment (start 178 78.0647) (end 177.6327 78.0647) (width 0.25) (layer F.Cu) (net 8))
 (segment (start 178 79.24) (end 178 78.0647) (width 0.25) (layer F.Cu) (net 8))
 (segment (start 177.5373 67.7153) (end 178 67.7153) (width 0.25) (layer B.Cu) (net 11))
 (segment (start 174.2353 71.0173) (end 177.5373 67.7153) (width 0.25) (layer B.Cu) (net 11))
 (segment (start 174.2353 71.4448) (end 174.2353 71.0173) (width 0.25) (layer B.Cu) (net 11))
 (segment (start 174.0201 71.66) (end 174.2353 71.4448) (width 0.25) (layer B.Cu) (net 11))
 (segment (start 173.26 71.66) (end 174.0201 71.66) (width 0.25) (layer B.Cu) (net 11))
 (segment (start 178 66.54) (end 178 67.7153) (width 0.25) (layer B.Cu) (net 11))
 (segment (start 178 69.08) (end 176.8247 69.08) (width 0.25) (layer B.Cu) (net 12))
 (segment (start 173.26 72.16) (end 174.2353 72.16) (width 0.25) (layer B.Cu) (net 12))
 (segment (start 176.8247 69.5706) (end 176.8247 69.08) (width 0.25) (layer B.Cu) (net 12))
 (segment (start 174.2353 72.16) (end 176.8247 69.5706) (width 0.25) (layer B.Cu) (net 12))
 (segment (start 174.2353 74.7475) (end 174.2353 74.66) (width 0.25) (layer B.Cu) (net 13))
 (segment (start 177.3914 77.9036) (end 174.2353 74.7475) (width 0.25) (layer B.Cu) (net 13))
 (segment (start 178.4798 77.9036) (end 177.3914 77.9036) (width 0.25) (layer B.Cu) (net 13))
 (segment (start 179.1776 77.2058) (end 178.4798 77.9036) (width 0.25) (layer B.Cu) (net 13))
 (segment (start 179.1776 73.6056) (end 179.1776 77.2058) (width 0.25) (layer B.Cu) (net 13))
 (segment (start 178.3673 72.7953) (end 179.1776 73.6056) (width 0.25) (layer B.Cu) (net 13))
 (segment (start 178 72.7953) (end 178.3673 72.7953) (width 0.25) (layer B.Cu) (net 13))
 (segment (start 178 71.62) (end 178 72.7953) (width 0.25) (layer B.Cu) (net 13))
 (segment (start 173.26 74.66) (end 174.2353 74.66) (width 0.25) (layer B.Cu) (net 13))
 (segment (start 176.3247 73.66) (end 173.26 73.66) (width 0.25) (layer B.Cu) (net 14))
 (segment (start 176.8247 74.16) (end 176.3247 73.66) (width 0.25) (layer B.Cu) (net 14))
 (segment (start 178 74.16) (end 176.8247 74.16) (width 0.25) (layer B.Cu) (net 14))
 (segment (start 178 76.7) (end 176.8247 76.7) (width 0.25) (layer B.Cu) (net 15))
 (segment (start 174.444 74.16) (end 173.26 74.16) (width 0.25) (layer B.Cu) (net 15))
 (segment (start 176.8247 76.5407) (end 174.444 74.16) (width 0.25) (layer B.Cu) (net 15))
 (segment (start 176.8247 76.7) (end 176.8247 76.5407) (width 0.25) (layer B.Cu) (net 15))
 (segment (start 168.46 97.5753) (end 168.46 102) (width 0.25) (layer F.Cu) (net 10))
 (segment (start 178 88.0353) (end 168.46 97.5753) (width 0.25) (layer F.Cu) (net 10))
 (segment (start 178 86.86) (end 178 88.0353) (width 0.25) (layer F.Cu) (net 10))
 (segment (start 169 51) (end 169 52.1753) (width 0.25) (layer B.Cu) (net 9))
 (segment (start 172.1391 78.16) (end 173.26 78.16) (width 0.25) (layer B.Cu) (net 9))
 (segment (start 171.6201 77.641) (end 172.1391 78.16) (width 0.25) (layer B.Cu) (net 9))
 (segment (start 171.6201 54.7954) (end 171.6201 77.641) (width 0.25) (layer B.Cu) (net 9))
 (segment (start 169 52.1753) (end 171.6201 54.7954) (width 0.25) (layer B.Cu) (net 9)))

